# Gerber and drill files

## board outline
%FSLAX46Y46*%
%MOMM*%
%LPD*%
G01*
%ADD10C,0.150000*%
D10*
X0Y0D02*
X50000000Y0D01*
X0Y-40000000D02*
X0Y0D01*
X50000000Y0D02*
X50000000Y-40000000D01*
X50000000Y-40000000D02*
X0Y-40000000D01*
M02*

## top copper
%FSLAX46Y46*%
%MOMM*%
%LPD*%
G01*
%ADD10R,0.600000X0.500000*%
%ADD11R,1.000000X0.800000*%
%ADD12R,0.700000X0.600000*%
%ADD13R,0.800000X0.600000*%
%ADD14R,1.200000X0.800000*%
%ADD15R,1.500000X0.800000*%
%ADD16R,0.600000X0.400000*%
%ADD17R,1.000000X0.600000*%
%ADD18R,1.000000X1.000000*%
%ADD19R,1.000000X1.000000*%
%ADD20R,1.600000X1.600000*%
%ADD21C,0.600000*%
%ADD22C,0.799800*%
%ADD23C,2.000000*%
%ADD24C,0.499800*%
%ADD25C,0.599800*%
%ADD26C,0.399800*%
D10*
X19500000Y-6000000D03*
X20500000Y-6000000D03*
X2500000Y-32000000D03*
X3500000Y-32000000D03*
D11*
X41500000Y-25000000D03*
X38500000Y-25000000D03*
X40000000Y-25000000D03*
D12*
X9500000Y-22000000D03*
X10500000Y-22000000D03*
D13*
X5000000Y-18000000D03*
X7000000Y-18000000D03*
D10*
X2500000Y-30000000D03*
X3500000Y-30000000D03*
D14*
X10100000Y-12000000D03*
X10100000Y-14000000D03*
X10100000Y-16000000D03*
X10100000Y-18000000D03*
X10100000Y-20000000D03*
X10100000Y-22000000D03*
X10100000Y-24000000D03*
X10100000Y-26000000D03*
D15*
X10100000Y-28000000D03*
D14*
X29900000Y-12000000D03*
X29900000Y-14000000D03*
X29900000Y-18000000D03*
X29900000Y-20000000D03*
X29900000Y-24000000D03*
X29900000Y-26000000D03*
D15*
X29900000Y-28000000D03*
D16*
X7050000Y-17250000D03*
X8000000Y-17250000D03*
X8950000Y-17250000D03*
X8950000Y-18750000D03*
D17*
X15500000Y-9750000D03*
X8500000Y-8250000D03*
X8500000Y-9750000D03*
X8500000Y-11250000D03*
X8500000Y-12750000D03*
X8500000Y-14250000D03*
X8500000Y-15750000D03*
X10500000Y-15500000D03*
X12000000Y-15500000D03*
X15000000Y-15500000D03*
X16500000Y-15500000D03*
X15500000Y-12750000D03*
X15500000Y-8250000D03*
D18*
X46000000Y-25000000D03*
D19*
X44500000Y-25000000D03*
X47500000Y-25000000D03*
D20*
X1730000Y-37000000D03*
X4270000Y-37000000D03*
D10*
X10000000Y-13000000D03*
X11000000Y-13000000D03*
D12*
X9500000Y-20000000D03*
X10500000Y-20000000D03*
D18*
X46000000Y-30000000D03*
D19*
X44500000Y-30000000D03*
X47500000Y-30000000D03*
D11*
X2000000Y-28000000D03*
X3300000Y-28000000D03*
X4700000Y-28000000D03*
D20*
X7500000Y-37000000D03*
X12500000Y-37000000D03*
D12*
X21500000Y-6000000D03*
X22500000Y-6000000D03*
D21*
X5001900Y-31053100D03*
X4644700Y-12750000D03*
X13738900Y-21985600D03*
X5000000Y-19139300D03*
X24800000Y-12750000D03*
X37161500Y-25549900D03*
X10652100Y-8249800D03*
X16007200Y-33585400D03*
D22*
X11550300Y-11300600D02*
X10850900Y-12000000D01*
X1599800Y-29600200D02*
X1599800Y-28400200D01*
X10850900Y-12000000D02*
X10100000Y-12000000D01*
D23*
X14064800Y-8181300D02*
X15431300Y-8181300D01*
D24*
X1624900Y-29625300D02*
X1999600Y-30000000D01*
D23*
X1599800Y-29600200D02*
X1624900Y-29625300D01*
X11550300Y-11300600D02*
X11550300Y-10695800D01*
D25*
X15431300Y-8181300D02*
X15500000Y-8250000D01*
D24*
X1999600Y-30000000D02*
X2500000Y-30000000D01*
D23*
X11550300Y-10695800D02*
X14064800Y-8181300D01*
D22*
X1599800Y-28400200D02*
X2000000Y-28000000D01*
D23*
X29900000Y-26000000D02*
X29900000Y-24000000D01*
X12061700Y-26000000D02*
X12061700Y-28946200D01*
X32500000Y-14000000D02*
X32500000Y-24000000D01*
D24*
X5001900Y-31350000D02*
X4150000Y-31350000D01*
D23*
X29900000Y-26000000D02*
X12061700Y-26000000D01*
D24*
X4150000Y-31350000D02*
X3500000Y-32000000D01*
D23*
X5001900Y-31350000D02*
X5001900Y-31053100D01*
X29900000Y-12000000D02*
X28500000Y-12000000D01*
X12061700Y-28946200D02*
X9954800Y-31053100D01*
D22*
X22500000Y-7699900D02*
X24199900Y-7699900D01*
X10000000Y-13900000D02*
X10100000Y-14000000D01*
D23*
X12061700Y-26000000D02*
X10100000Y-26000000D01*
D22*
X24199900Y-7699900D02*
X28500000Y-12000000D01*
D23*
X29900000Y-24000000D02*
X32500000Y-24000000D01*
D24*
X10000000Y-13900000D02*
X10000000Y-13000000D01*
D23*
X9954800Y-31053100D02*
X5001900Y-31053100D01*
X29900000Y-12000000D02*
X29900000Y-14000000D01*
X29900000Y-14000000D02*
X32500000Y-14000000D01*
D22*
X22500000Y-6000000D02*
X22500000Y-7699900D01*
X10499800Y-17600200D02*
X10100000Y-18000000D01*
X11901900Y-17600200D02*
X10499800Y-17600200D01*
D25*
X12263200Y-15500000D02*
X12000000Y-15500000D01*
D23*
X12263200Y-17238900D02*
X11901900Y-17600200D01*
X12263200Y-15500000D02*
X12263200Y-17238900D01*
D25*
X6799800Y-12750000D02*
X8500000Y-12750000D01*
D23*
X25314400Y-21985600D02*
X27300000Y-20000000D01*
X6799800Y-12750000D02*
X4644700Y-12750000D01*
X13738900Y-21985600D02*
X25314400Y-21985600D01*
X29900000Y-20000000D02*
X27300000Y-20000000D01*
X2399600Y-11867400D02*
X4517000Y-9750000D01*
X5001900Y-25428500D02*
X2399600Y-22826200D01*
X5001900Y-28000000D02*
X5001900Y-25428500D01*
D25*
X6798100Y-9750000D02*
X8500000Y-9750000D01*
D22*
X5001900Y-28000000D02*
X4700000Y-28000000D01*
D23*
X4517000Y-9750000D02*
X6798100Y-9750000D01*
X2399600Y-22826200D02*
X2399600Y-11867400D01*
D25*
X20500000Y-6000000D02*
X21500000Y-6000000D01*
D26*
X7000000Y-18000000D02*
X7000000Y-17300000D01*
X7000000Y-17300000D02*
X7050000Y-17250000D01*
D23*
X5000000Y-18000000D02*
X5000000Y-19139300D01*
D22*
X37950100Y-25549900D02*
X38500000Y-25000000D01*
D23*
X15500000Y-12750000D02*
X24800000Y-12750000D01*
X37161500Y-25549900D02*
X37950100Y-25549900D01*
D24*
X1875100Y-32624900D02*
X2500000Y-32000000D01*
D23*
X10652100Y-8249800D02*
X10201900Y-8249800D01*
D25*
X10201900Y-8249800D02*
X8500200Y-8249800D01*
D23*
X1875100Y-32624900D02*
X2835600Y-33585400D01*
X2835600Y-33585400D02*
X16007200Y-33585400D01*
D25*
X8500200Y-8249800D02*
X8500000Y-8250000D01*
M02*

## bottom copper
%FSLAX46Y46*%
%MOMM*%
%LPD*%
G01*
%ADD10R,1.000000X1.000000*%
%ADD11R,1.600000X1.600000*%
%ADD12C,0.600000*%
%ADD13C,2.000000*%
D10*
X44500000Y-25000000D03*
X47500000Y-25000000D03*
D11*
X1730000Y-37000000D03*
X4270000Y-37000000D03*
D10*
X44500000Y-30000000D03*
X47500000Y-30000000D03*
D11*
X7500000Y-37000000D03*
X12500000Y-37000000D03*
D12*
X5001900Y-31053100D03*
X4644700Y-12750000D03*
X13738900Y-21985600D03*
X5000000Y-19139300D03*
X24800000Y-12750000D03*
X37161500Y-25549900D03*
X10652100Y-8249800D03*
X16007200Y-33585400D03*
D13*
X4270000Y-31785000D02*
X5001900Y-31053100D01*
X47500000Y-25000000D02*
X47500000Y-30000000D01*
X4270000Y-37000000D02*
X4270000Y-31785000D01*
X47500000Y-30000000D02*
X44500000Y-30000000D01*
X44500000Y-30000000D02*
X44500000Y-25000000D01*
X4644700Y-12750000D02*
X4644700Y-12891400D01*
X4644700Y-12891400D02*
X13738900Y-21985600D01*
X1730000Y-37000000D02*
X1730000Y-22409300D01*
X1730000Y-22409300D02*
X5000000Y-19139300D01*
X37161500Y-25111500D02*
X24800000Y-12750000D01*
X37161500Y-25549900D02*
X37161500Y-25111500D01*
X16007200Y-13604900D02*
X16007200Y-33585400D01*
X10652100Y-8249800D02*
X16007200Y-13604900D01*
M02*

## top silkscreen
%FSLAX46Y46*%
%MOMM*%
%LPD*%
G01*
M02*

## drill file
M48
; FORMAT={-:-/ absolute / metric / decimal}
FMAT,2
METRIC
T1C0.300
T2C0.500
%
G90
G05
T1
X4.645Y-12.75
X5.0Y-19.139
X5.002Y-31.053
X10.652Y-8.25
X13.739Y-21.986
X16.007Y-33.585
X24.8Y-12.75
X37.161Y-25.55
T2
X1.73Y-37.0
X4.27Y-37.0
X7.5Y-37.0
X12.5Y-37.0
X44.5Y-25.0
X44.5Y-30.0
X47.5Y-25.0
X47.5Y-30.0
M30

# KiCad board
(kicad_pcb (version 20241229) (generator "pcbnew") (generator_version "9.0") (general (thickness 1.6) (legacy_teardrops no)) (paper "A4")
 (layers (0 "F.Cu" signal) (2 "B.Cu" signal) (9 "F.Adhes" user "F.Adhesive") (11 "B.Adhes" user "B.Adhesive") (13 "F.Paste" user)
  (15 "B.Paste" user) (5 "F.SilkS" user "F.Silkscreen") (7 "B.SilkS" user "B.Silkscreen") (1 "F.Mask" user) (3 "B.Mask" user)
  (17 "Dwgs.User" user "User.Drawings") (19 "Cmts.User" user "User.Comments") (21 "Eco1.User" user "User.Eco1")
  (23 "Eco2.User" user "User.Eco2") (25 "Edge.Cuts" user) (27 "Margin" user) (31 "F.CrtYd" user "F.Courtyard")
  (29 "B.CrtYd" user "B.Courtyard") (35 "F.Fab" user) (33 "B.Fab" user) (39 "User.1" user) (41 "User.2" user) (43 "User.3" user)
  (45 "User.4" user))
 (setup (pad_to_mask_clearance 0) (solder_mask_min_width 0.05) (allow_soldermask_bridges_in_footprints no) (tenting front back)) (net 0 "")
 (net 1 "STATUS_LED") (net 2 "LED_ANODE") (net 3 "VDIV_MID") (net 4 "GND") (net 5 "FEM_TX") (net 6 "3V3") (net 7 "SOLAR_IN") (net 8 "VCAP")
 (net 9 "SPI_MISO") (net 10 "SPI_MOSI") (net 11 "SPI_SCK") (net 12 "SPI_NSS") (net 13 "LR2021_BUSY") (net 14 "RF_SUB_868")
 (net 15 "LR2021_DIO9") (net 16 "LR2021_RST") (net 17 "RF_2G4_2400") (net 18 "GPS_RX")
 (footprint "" (layer "F.Cu") (at 20 6)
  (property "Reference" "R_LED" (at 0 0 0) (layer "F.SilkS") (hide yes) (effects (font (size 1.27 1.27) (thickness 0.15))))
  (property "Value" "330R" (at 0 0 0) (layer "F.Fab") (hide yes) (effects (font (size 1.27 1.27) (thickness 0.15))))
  (pad "1" smd rect (at -0.5 0) (size 0.6 0.5) (layers "F.Cu" "F.Mask") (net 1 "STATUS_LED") (thermal_bridge_angle 45))
  (pad "2" smd rect (at 0.5 0) (size 0.6 0.5) (layers "F.Cu" "F.Mask") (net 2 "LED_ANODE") (thermal_bridge_angle 45)))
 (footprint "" (layer "F.Cu") (at 3 32)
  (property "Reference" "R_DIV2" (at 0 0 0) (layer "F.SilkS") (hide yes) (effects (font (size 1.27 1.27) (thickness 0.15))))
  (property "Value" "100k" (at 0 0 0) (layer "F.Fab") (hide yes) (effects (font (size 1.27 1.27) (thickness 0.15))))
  (pad "1" smd rect (at -0.5 0) (size 0.6 0.5) (layers "F.Cu" "F.Mask") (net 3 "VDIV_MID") (thermal_bridge_angle 45))
  (pad "2" smd rect (at 0.5 0) (size 0.6 0.5) (layers "F.Cu" "F.Mask") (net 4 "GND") (thermal_bridge_angle 45)))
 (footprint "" (layer "F.Cu") (at 40 25)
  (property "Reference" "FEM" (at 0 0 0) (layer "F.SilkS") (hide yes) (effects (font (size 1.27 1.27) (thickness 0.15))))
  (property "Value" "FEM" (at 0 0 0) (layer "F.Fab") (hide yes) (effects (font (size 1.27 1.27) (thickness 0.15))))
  (pad "GND" smd rect (at 1.5 0) (size 1 0.8) (layers "F.Cu" "F.Mask") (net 4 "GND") (thermal_bridge_angle 45))
  (pad "TX" smd rect (at -1.5 0) (size 1 0.8) (layers "F.Cu" "F.Mask") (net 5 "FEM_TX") (thermal_bridge_angle 45))
  (pad "VCC" smd rect (at 0 0) (size 1 0.8) (layers "F.Cu" "F.Mask") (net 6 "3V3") (thermal_bridge_angle 45)))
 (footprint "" (layer "F.Cu") (at 10 22)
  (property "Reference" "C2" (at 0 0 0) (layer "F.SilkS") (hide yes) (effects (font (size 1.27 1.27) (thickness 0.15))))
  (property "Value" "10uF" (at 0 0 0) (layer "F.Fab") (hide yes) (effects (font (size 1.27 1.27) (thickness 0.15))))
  (pad "1" smd rect (at -0.5 0) (size 0.7 0.6) (layers "F.Cu" "F.Mask") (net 6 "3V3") (thermal_bridge_angle 45))
  (pad "2" smd rect (at 0.5 0) (size 0.7 0.6) (layers "F.Cu" "F.Mask") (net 4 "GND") (thermal_bridge_angle 45)))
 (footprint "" (layer "F.Cu") (at 6 18)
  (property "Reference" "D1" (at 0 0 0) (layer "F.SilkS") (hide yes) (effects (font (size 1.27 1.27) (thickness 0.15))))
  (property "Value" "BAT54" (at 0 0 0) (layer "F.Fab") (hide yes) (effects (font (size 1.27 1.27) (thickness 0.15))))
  (pad "A" smd rect (at -1 0) (size 0.8 0.6) (layers "F.Cu" "F.Mask") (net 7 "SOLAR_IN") (thermal_bridge_angle 45))
  (pad "K" smd rect (at 1 0) (size 0.8 0.6) (layers "F.Cu" "F.Mask") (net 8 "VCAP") (thermal_bridge_angle 45)))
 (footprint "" (layer "F.Cu") (at 3 30)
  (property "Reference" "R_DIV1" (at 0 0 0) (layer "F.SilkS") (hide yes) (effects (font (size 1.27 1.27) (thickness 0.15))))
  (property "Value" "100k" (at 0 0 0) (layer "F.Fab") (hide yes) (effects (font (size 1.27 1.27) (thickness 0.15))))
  (pad "1" smd rect (at -0.5 0) (size 0.6 0.5) (layers "F.Cu" "F.Mask") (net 6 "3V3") (thermal_bridge_angle 45))
  (pad "2" smd rect (at 0.5 0) (size 0.6 0.5) (layers "F.Cu" "F.Mask") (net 3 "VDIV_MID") (thermal_bridge_angle 45)))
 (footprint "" (layer "F.Cu") (at 20 20)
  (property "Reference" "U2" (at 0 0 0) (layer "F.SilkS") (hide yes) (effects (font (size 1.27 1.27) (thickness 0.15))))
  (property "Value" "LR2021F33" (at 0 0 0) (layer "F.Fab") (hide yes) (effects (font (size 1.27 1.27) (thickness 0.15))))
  (pad "1" smd rect (at -9.9 -8) (size 1.2 0.8) (layers "F.Cu" "F.Mask") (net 6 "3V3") (thermal_bridge_angle 45))
  (pad "2" smd rect (at -9.9 -6) (size 1.2 0.8) (layers "F.Cu" "F.Mask") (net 4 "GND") (thermal_bridge_angle 45))
  (pad "3" smd rect (at -9.9 -4) (size 1.2 0.8) (layers "F.Cu" "F.Mask") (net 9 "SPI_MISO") (thermal_bridge_angle 45))
  (pad "4" smd rect (at -9.9 -2) (size 1.2 0.8) (layers "F.Cu" "F.Mask") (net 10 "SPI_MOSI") (thermal_bridge_angle 45))
  (pad "5" smd rect (at -9.9 0) (size 1.2 0.8) (layers "F.Cu" "F.Mask") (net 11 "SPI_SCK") (thermal_bridge_angle 45))
  (pad "6" smd rect (at -9.9 2) (size 1.2 0.8) (layers "F.Cu" "F.Mask") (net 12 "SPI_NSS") (thermal_bridge_angle 45))
  (pad "7" smd rect (at -9.9 4) (size 1.2 0.8) (layers "F.Cu" "F.Mask") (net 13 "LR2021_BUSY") (thermal_bridge_angle 45))
  (pad "8" smd rect (at -9.9 6) (size 1.2 0.8) (layers "F.Cu" "F.Mask") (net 4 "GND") (thermal_bridge_angle 45))
  (pad "9" smd rect (at -9.9 8) (size 1.5 0.8) (layers "F.Cu" "F.Mask") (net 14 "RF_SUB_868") (thermal_bridge_angle 45))
  (pad "10" smd rect (at 9.9 -8) (size 1.2 0.8) (layers "F.Cu" "F.Mask") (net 4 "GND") (thermal_bridge_angle 45))
  (pad "11" smd rect (at 9.9 -6) (size 1.2 0.8) (layers "F.Cu" "F.Mask") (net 4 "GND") (thermal_bridge_angle 45))
  (pad "13" smd rect (at 9.9 -2) (size 1.2 0.8) (layers "F.Cu" "F.Mask") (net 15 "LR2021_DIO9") (thermal_bridge_angle 45))
  (pad "14" smd rect (at 9.9 0) (size 1.2 0.8) (layers "F.Cu" "F.Mask") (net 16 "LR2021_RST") (thermal_bridge_angle 45))
  (pad "16" smd rect (at 9.9 4) (size 1.2 0.8) (layers "F.Cu" "F.Mask") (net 4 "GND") (thermal_bridge_angle 45))
  (pad "17" smd rect (at 9.9 6) (size 1.2 0.8) (layers "F.Cu" "F.Mask") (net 4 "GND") (thermal_bridge_angle 45))
  (pad "18" smd rect (at 9.9 8) (size 1.5 0.8) (layers "F.Cu" "F.Mask") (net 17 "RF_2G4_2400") (thermal_bridge_angle 45)))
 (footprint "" (layer "F.Cu") (at 8 18)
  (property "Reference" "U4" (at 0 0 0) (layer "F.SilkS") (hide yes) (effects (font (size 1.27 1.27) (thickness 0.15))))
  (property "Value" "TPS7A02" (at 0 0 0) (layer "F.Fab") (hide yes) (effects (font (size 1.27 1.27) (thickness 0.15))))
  (pad "1" smd rect (at -0.95 -0.75) (size 0.6 0.4) (layers "F.Cu" "F.Mask") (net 8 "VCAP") (thermal_bridge_angle 45))
  (pad "2" smd rect (at 0 -0.75) (size 0.6 0.4) (layers "F.Cu" "F.Mask") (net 4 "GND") (thermal_bridge_angle 45))
  (pad "3" smd rect (at 0.95 -0.75) (size 0.6 0.4) (layers "F.Cu" "F.Mask") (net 8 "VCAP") (thermal_bridge_angle 45))
  (pad "4" smd rect (at 0.95 0.75) (size 0.6 0.4) (layers "F.Cu" "F.Mask") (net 6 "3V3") (thermal_bridge_angle 45)))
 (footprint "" (layer "F.Cu") (at 12 12)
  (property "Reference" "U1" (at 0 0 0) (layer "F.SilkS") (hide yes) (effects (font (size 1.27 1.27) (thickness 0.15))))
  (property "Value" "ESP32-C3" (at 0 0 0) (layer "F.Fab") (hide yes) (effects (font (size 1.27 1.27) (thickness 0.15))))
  (pad "GND" smd rect (at 3.5 -2.25) (size 1 0.6) (layers "F.Cu" "F.Mask") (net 4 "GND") (thermal_bridge_angle 45))
  (pad "GPIO0" smd rect (at -3.5 -3.75) (size 1 0.6) (layers "F.Cu" "F.Mask") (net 3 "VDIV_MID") (thermal_bridge_angle 45))
  (pad "GPIO1" smd rect (at -3.5 -2.25) (size 1 0.6) (layers "F.Cu" "F.Mask") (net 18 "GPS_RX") (thermal_bridge_angle 45))
  (pad "GPIO2" smd rect (at -3.5 -0.75) (size 1 0.6) (layers "F.Cu" "F.Mask") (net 9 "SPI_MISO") (thermal_bridge_angle 45))
  (pad "GPIO3" smd rect (at -3.5 0.75) (size 1 0.6) (layers "F.Cu" "F.Mask") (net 16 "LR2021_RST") (thermal_bridge_angle 45))
  (pad "GPIO4" smd rect (at -3.5 2.25) (size 1 0.6) (layers "F.Cu" "F.Mask") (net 13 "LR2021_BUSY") (thermal_bridge_angle 45))
  (pad "GPIO5" smd rect (at -3.5 3.75) (size 1 0.6) (layers "F.Cu" "F.Mask") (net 15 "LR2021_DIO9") (thermal_bridge_angle 45))
  (pad "GPIO6" smd rect (at -1.5 3.5) (size 1 0.6) (layers "F.Cu" "F.Mask") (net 11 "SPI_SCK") (thermal_bridge_angle 45))
  (pad "GPIO7" smd rect (at 0 3.5) (size 1 0.6) (layers "F.Cu" "F.Mask") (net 10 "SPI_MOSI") (thermal_bridge_angle 45))
  (pad "GPIO9" smd rect (at 3 3.5) (size 1 0.6) (layers "F.Cu" "F.Mask") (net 1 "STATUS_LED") (thermal_bridge_angle 45))
  (pad "GPIO10" smd rect (at 4.5 3.5) (size 1 0.6) (layers "F.Cu" "F.Mask") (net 12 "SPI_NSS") (thermal_bridge_angle 45))
  (pad "GPIO19" smd rect (at 3.5 0.75) (size 1 0.6) (layers "F.Cu" "F.Mask") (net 5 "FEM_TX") (thermal_bridge_angle 45))
  (pad "VCC" smd rect (at 3.5 -3.75) (size 1 0.6) (layers "F.Cu" "F.Mask") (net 6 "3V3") (thermal_bridge_angle 45)))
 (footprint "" (layer "F.Cu") (at 46 25)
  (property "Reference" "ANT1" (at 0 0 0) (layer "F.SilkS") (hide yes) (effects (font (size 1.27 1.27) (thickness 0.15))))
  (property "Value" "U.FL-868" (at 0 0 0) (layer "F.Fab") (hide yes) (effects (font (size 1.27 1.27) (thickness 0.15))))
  (pad "1" smd rect (at 0 0) (size 1 1) (layers "F.Cu" "F.Mask") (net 14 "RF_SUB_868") (thermal_bridge_angle 45))
  (pad "2" thru_hole rect (at -1.5 0) (size 1 1) (drill 0.5) (layers "*.Cu" "*.Mask") (remove_unused_layers no) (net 4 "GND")
   (thermal_bridge_angle 45))
  (pad "3" thru_hole rect (at 1.5 0) (size 1 1) (drill 0.5) (layers "*.Cu" "*.Mask") (remove_unused_layers no) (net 4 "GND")
   (thermal_bridge_angle 45)))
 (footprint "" (layer "F.Cu") (at 3 37)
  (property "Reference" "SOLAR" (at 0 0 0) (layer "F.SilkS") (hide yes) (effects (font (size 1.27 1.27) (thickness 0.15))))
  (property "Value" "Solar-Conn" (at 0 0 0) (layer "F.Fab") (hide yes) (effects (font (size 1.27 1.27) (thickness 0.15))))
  (pad "1" thru_hole rect (at -1.27 0) (size 1.6 1.6) (drill 0.5) (layers "*.Cu" "*.Mask") (remove_unused_layers no) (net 7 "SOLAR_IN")
   (thermal_bridge_angle 45))
  (pad "2" thru_hole rect (at 1.27 0) (size 1.6 1.6) (drill 0.5) (layers "*.Cu" "*.Mask") (remove_unused_layers no) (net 4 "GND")
   (thermal_bridge_angle 45)))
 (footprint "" (layer "F.Cu") (at 10.5 13)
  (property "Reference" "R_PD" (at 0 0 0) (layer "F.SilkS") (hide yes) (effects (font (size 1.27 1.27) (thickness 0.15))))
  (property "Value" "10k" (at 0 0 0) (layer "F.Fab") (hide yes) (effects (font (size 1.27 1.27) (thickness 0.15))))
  (pad "1" smd rect (at -0.5 0) (size 0.6 0.5) (layers "F.Cu" "F.Mask") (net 4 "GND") (thermal_bridge_angle 45))
  (pad "2" smd rect (at 0.5 0) (size 0.6 0.5) (layers "F.Cu" "F.Mask") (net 9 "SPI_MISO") (thermal_bridge_angle 45)))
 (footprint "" (layer "F.Cu") (at 10 20)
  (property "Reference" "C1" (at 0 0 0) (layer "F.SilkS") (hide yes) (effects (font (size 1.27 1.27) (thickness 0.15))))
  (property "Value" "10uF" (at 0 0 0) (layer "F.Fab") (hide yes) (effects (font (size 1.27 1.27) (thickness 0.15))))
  (pad "1" smd rect (at -0.5 0) (size 0.7 0.6) (layers "F.Cu" "F.Mask") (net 8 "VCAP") (thermal_bridge_angle 45))
  (pad "2" smd rect (at 0.5 0) (size 0.7 0.6) (layers "F.Cu" "F.Mask") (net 4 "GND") (thermal_bridge_angle 45)))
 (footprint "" (layer "F.Cu") (at 46 30)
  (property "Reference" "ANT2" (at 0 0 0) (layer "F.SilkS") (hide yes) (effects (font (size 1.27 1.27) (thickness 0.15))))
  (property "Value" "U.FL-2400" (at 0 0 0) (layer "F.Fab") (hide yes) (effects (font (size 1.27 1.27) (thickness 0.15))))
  (pad "1" smd rect (at 0 0) (size 1 1) (layers "F.Cu" "F.Mask") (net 17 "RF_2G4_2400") (thermal_bridge_angle 45))
  (pad "2" thru_hole rect (at -1.5 0) (size 1 1) (drill 0.5) (layers "*.Cu" "*.Mask") (remove_unused_layers no) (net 4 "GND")
   (thermal_bridge_angle 45))
  (pad "3" thru_hole rect (at 1.5 0) (size 1 1) (drill 0.5) (layers "*.Cu" "*.Mask") (remove_unused_layers no) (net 4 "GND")
   (thermal_bridge_angle 45)))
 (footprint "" (layer "F.Cu") (at 4 28)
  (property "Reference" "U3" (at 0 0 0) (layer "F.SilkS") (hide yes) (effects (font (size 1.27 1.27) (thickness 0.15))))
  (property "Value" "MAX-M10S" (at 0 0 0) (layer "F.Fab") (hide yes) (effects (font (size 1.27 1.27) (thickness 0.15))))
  (pad "1" smd rect (at -2 0) (size 1 0.8) (layers "F.Cu" "F.Mask") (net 6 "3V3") (thermal_bridge_angle 45))
  (pad "2" smd rect (at -0.7 0) (size 1 0.8) (layers "F.Cu" "F.Mask") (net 4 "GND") (thermal_bridge_angle 45))
  (pad "3" smd rect (at 0.7 0) (size 1 0.8) (layers "F.Cu" "F.Mask") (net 18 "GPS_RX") (thermal_bridge_angle 45)))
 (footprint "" (layer "F.Cu") (at 10 37)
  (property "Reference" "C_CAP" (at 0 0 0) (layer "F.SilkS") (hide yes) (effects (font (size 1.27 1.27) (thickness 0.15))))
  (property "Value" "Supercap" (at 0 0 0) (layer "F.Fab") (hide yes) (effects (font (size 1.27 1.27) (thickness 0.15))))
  (pad "1" thru_hole rect (at -2.5 0) (size 1.6 1.6) (drill 0.5) (layers "*.Cu" "*.Mask") (remove_unused_layers no) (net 8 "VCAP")
   (thermal_bridge_angle 45))
  (pad "2" thru_hole rect (at 2.5 0) (size 1.6 1.6) (drill 0.5) (layers "*.Cu" "*.Mask") (remove_unused_layers no) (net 4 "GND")
   (thermal_bridge_angle 45)))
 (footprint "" (layer "F.Cu") (at 22 6)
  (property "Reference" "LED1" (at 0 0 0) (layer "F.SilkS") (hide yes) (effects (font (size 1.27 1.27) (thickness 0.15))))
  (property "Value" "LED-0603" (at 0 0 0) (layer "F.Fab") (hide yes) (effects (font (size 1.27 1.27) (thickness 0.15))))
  (pad "A" smd rect (at -0.5 0) (size 0.7 0.6) (layers "F.Cu" "F.Mask") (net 2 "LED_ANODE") (thermal_bridge_angle 45))
  (pad "K" smd rect (at 0.5 0) (size 0.7 0.6) (layers "F.Cu" "F.Mask") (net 4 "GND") (thermal_bridge_angle 45)))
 (gr_line (start 0 0) (end 50 0) (stroke (width 0.15) (type default)) (layer "Edge.Cuts"))
 (gr_line (start 0 40) (end 0 0) (stroke (width 0.15) (type default)) (layer "Edge.Cuts"))
 (gr_line (start 50 0) (end 50 40) (stroke (width 0.15) (type default)) (layer "Edge.Cuts"))
 (gr_line (start 50 40) (end 0 40) (stroke (width 0.15) (type default)) (layer "Edge.Cuts"))
 (segment (start 11.5503 11.3006) (end 10.8509 12) (width 0.7998) (layer "F.Cu") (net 6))
 (segment (start 1.5998 29.6002) (end 1.5998 28.4002) (width 0.7998) (layer "F.Cu") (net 6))
 (segment (start 10.8509 12) (end 10.1 12) (width 0.7998) (layer "F.Cu") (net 6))
 (segment (start 14.0648 8.1813) (end 15.4313 8.1813) (width 2) (layer "F.Cu") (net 6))
 (segment (start 1.6249 29.6253) (end 1.9996 30) (width 0.4998) (layer "F.Cu") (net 6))
 (segment (start 1.5998 29.6002) (end 1.6249 29.6253) (width 2) (layer "F.Cu") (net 6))
 (segment (start 11.5503 11.3006) (end 11.5503 10.6958) (width 2) (layer "F.Cu") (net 6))
 (segment (start 15.4313 8.1813) (end 15.5 8.25) (width 0.5998) (layer "F.Cu") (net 6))
 (segment (start 1.9996 30) (end 2.5 30) (width 0.4998) (layer "F.Cu") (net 6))
 (segment (start 11.5503 10.6958) (end 14.0648 8.1813) (width 2) (layer "F.Cu") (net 6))
 (segment (start 1.5998 28.4002) (end 2 28) (width 0.7998) (layer "F.Cu") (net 6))
 (segment (start 29.9 26) (end 29.9 24) (width 2) (layer "F.Cu") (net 4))
 (segment (start 12.0617 26) (end 12.0617 28.9462) (width 2) (layer "F.Cu") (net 4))
 (segment (start 32.5 14) (end 32.5 24) (width 2) (layer "F.Cu") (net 4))
 (segment (start 5.0019 31.35) (end 4.15 31.35) (width 0.4998) (layer "F.Cu") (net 4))
 (segment (start 29.9 26) (end 12.0617 26) (width 2) (layer "F.Cu") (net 4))
 (segment (start 4.15 31.35) (end 3.5 32) (width 0.4998) (layer "F.Cu") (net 4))
 (segment (start 5.0019 31.35) (end 5.0019 31.0531) (width 2) (layer "F.Cu") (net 4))
 (segment (start 29.9 12) (end 28.5 12) (width 2) (layer "F.Cu") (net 4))
 (segment (start 12.0617 28.9462) (end 9.9548 31.0531) (width 2) (layer "F.Cu") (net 4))
 (segment (start 22.5 7.6999) (end 24.1999 7.6999) (width 0.7998) (layer "F.Cu") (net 4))
 (segment (start 10 13.9) (end 10.1 14) (width 0.7998) (layer "F.Cu") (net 4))
 (segment (start 12.0617 26) (end 10.1 26) (width 2) (layer "F.Cu") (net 4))
 (segment (start 24.1999 7.6999) (end 28.5 12) (width 0.7998) (layer "F.Cu") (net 4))
 (segment (start 29.9 24) (end 32.5 24) (width 2) (layer "F.Cu") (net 4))
 (segment (start 10 13.9) (end 10 13) (width 0.4998) (layer "F.Cu") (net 4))
 (segment (start 9.9548 31.0531) (end 5.0019 31.0531) (width 2) (layer "F.Cu") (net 4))
 (segment (start 29.9 12) (end 29.9 14) (width 2) (layer "F.Cu") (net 4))
 (segment (start 29.9 14) (end 32.5 14) (width 2) (layer "F.Cu") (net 4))
 (segment (start 22.5 6) (end 22.5 7.6999) (width 0.7998) (layer "F.Cu") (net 4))
 (via (at 5.0019 31.0531) (size 0.6) (drill 0.3) (layers "F.Cu" "B.Cu") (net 4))
 (segment (start 4.27 31.785) (end 5.0019 31.0531) (width 2) (layer "B.Cu") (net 4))
 (segment (start 47.5 25) (end 47.5 30) (width 2) (layer "B.Cu") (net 4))
 (segment (start 4.27 37) (end 4.27 31.785) (width 2) (layer "B.Cu") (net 4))
 (segment (start 47.5 30) (end 44.5 30) (width 2) (layer "B.Cu") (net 4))
 (segment (start 44.5 30) (end 44.5 25) (width 2) (layer "B.Cu") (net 4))
 (segment (start 10.4998 17.6002) (end 10.1 18) (width 0.7998) (layer "F.Cu") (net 10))
 (segment (start 11.9019 17.6002) (end 10.4998 17.6002) (width 0.7998) (layer "F.Cu") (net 10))
 (segment (start 12.2632 15.5) (end 12 15.5) (width 0.5998) (layer "F.Cu") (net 10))
 (segment (start 12.2632 17.2389) (end 11.9019 17.6002) (width 2) (layer "F.Cu") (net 10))
 (segment (start 12.2632 15.5) (end 12.2632 17.2389) (width 2) (layer "F.Cu") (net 10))
 (segment (start 6.7998 12.75) (end 8.5 12.75) (width 0.5998) (layer "F.Cu") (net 16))
 (segment (start 25.3144 21.9856) (end 27.3 20) (width 2) (layer "F.Cu") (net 16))
 (segment (start 6.7998 12.75) (end 4.6447 12.75) (width 2) (layer "F.Cu") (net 16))
 (segment (start 13.7389 21.9856) (end 25.3144 21.9856) (width 2) (layer "F.Cu") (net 16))
 (segment (start 29.9 20) (end 27.3 20) (width 2) (layer "F.Cu") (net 16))
 (via (at 4.6447 12.75) (size 0.6) (drill 0.3) (layers "F.Cu" "B.Cu") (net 16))
 (via (at 13.7389 21.9856) (size 0.6) (drill 0.3) (layers "F.Cu" "B.Cu") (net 16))
 (segment (start 4.6447 12.75) (end 4.6447 12.8914) (width 2) (layer "B.Cu") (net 16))
 (segment (start 4.6447 12.8914) (end 13.7389 21.9856) (width 2) (layer "B.Cu") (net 16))
 (segment (start 2.3996 11.8674) (end 4.517 9.75) (width 2) (layer "F.Cu") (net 18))
 (segment (start 5.0019 25.4285) (end 2.3996 22.8262) (width 2) (layer "F.Cu") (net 18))
 (segment (start 5.0019 28) (end 5.0019 25.4285) (width 2) (layer "F.Cu") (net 18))
 (segment (start 6.7981 9.75) (end 8.5 9.75) (width 0.5998) (layer "F.Cu") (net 18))
 (segment (start 5.0019 28) (end 4.7 28) (width 0.7998) (layer "F.Cu") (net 18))
 (segment (start 4.517 9.75) (end 6.7981 9.75) (width 2) (layer "F.Cu") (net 18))
 (segment (start 2.3996 22.8262) (end 2.3996 11.8674) (width 2) (layer "F.Cu") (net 18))
 (segment (start 20.5 6) (end 21.5 6) (width 0.5998) (layer "F.Cu") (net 2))
 (segment (start 7 18) (end 7 17.3) (width 0.3998) (layer "F.Cu") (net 8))
 (segment (start 7 17.3) (end 7.05 17.25) (width 0.3998) (layer "F.Cu") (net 8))
 (segment (start 5 18) (end 5 19.1393) (width 2) (layer "F.Cu") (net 7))
 (via (at 5 19.1393) (size 0.6) (drill 0.3) (layers "F.Cu" "B.Cu") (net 7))
 (segment (start 1.73 37) (end 1.73 22.4093) (width 2) (layer "B.Cu") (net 7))
 (segment (start 1.73 22.4093) (end 5 19.1393) (width 2) (layer "B.Cu") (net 7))
 (segment (start 37.9501 25.5499) (end 38.5 25) (width 0.7998) (layer "F.Cu") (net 5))
 (segment (start 15.5 12.75) (end 24.8 12.75) (width 2) (layer "F.Cu") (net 5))
 (segment (start 37.1615 25.5499) (end 37.9501 25.5499) (width 2) (layer "F.Cu") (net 5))
 (via (at 24.8 12.75) (size 0.6) (drill 0.3) (layers "F.Cu" "B.Cu") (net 5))
 (via (at 37.1615 25.5499) (size 0.6) (drill 0.3) (layers "F.Cu" "B.Cu") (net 5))
 (segment (start 37.1615 25.1115) (end 24.8 12.75) (width 2) (layer "B.Cu") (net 5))
 (segment (start 37.1615 25.5499) (end 37.1615 25.1115) (width 2) (layer "B.Cu") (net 5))
 (segment (start 1.8751 32.6249) (end 2.5 32) (width 0.4998) (layer "F.Cu") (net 3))
 (segment (start 10.6521 8.2498) (end 10.2019 8.2498) (width 2) (layer "F.Cu") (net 3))
 (segment (start 10.2019 8.2498) (end 8.5002 8.2498) (width 0.5998) (layer "F.Cu") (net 3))
 (segment (start 1.8751 32.6249) (end 2.8356 33.5854) (width 2) (layer "F.Cu") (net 3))
 (segment (start 2.8356 33.5854) (end 16.0072 33.5854) (width 2) (layer "F.Cu") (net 3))
 (segment (start 8.5002 8.2498) (end 8.5 8.25) (width 0.5998) (layer "F.Cu") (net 3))
 (via (at 10.6521 8.2498) (size 0.6) (drill 0.3) (layers "F.Cu" "B.Cu") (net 3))
 (via (at 16.0072 33.5854) (size 0.6) (drill 0.3) (layers "F.Cu" "B.Cu") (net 3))
 (segment (start 16.0072 13.6049) (end 16.0072 33.5854) (width 2) (layer "B.Cu") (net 3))
 (segment (start 10.6521 8.2498) (end 16.0072 13.6049) (width 2) (layer "B.Cu") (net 3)))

